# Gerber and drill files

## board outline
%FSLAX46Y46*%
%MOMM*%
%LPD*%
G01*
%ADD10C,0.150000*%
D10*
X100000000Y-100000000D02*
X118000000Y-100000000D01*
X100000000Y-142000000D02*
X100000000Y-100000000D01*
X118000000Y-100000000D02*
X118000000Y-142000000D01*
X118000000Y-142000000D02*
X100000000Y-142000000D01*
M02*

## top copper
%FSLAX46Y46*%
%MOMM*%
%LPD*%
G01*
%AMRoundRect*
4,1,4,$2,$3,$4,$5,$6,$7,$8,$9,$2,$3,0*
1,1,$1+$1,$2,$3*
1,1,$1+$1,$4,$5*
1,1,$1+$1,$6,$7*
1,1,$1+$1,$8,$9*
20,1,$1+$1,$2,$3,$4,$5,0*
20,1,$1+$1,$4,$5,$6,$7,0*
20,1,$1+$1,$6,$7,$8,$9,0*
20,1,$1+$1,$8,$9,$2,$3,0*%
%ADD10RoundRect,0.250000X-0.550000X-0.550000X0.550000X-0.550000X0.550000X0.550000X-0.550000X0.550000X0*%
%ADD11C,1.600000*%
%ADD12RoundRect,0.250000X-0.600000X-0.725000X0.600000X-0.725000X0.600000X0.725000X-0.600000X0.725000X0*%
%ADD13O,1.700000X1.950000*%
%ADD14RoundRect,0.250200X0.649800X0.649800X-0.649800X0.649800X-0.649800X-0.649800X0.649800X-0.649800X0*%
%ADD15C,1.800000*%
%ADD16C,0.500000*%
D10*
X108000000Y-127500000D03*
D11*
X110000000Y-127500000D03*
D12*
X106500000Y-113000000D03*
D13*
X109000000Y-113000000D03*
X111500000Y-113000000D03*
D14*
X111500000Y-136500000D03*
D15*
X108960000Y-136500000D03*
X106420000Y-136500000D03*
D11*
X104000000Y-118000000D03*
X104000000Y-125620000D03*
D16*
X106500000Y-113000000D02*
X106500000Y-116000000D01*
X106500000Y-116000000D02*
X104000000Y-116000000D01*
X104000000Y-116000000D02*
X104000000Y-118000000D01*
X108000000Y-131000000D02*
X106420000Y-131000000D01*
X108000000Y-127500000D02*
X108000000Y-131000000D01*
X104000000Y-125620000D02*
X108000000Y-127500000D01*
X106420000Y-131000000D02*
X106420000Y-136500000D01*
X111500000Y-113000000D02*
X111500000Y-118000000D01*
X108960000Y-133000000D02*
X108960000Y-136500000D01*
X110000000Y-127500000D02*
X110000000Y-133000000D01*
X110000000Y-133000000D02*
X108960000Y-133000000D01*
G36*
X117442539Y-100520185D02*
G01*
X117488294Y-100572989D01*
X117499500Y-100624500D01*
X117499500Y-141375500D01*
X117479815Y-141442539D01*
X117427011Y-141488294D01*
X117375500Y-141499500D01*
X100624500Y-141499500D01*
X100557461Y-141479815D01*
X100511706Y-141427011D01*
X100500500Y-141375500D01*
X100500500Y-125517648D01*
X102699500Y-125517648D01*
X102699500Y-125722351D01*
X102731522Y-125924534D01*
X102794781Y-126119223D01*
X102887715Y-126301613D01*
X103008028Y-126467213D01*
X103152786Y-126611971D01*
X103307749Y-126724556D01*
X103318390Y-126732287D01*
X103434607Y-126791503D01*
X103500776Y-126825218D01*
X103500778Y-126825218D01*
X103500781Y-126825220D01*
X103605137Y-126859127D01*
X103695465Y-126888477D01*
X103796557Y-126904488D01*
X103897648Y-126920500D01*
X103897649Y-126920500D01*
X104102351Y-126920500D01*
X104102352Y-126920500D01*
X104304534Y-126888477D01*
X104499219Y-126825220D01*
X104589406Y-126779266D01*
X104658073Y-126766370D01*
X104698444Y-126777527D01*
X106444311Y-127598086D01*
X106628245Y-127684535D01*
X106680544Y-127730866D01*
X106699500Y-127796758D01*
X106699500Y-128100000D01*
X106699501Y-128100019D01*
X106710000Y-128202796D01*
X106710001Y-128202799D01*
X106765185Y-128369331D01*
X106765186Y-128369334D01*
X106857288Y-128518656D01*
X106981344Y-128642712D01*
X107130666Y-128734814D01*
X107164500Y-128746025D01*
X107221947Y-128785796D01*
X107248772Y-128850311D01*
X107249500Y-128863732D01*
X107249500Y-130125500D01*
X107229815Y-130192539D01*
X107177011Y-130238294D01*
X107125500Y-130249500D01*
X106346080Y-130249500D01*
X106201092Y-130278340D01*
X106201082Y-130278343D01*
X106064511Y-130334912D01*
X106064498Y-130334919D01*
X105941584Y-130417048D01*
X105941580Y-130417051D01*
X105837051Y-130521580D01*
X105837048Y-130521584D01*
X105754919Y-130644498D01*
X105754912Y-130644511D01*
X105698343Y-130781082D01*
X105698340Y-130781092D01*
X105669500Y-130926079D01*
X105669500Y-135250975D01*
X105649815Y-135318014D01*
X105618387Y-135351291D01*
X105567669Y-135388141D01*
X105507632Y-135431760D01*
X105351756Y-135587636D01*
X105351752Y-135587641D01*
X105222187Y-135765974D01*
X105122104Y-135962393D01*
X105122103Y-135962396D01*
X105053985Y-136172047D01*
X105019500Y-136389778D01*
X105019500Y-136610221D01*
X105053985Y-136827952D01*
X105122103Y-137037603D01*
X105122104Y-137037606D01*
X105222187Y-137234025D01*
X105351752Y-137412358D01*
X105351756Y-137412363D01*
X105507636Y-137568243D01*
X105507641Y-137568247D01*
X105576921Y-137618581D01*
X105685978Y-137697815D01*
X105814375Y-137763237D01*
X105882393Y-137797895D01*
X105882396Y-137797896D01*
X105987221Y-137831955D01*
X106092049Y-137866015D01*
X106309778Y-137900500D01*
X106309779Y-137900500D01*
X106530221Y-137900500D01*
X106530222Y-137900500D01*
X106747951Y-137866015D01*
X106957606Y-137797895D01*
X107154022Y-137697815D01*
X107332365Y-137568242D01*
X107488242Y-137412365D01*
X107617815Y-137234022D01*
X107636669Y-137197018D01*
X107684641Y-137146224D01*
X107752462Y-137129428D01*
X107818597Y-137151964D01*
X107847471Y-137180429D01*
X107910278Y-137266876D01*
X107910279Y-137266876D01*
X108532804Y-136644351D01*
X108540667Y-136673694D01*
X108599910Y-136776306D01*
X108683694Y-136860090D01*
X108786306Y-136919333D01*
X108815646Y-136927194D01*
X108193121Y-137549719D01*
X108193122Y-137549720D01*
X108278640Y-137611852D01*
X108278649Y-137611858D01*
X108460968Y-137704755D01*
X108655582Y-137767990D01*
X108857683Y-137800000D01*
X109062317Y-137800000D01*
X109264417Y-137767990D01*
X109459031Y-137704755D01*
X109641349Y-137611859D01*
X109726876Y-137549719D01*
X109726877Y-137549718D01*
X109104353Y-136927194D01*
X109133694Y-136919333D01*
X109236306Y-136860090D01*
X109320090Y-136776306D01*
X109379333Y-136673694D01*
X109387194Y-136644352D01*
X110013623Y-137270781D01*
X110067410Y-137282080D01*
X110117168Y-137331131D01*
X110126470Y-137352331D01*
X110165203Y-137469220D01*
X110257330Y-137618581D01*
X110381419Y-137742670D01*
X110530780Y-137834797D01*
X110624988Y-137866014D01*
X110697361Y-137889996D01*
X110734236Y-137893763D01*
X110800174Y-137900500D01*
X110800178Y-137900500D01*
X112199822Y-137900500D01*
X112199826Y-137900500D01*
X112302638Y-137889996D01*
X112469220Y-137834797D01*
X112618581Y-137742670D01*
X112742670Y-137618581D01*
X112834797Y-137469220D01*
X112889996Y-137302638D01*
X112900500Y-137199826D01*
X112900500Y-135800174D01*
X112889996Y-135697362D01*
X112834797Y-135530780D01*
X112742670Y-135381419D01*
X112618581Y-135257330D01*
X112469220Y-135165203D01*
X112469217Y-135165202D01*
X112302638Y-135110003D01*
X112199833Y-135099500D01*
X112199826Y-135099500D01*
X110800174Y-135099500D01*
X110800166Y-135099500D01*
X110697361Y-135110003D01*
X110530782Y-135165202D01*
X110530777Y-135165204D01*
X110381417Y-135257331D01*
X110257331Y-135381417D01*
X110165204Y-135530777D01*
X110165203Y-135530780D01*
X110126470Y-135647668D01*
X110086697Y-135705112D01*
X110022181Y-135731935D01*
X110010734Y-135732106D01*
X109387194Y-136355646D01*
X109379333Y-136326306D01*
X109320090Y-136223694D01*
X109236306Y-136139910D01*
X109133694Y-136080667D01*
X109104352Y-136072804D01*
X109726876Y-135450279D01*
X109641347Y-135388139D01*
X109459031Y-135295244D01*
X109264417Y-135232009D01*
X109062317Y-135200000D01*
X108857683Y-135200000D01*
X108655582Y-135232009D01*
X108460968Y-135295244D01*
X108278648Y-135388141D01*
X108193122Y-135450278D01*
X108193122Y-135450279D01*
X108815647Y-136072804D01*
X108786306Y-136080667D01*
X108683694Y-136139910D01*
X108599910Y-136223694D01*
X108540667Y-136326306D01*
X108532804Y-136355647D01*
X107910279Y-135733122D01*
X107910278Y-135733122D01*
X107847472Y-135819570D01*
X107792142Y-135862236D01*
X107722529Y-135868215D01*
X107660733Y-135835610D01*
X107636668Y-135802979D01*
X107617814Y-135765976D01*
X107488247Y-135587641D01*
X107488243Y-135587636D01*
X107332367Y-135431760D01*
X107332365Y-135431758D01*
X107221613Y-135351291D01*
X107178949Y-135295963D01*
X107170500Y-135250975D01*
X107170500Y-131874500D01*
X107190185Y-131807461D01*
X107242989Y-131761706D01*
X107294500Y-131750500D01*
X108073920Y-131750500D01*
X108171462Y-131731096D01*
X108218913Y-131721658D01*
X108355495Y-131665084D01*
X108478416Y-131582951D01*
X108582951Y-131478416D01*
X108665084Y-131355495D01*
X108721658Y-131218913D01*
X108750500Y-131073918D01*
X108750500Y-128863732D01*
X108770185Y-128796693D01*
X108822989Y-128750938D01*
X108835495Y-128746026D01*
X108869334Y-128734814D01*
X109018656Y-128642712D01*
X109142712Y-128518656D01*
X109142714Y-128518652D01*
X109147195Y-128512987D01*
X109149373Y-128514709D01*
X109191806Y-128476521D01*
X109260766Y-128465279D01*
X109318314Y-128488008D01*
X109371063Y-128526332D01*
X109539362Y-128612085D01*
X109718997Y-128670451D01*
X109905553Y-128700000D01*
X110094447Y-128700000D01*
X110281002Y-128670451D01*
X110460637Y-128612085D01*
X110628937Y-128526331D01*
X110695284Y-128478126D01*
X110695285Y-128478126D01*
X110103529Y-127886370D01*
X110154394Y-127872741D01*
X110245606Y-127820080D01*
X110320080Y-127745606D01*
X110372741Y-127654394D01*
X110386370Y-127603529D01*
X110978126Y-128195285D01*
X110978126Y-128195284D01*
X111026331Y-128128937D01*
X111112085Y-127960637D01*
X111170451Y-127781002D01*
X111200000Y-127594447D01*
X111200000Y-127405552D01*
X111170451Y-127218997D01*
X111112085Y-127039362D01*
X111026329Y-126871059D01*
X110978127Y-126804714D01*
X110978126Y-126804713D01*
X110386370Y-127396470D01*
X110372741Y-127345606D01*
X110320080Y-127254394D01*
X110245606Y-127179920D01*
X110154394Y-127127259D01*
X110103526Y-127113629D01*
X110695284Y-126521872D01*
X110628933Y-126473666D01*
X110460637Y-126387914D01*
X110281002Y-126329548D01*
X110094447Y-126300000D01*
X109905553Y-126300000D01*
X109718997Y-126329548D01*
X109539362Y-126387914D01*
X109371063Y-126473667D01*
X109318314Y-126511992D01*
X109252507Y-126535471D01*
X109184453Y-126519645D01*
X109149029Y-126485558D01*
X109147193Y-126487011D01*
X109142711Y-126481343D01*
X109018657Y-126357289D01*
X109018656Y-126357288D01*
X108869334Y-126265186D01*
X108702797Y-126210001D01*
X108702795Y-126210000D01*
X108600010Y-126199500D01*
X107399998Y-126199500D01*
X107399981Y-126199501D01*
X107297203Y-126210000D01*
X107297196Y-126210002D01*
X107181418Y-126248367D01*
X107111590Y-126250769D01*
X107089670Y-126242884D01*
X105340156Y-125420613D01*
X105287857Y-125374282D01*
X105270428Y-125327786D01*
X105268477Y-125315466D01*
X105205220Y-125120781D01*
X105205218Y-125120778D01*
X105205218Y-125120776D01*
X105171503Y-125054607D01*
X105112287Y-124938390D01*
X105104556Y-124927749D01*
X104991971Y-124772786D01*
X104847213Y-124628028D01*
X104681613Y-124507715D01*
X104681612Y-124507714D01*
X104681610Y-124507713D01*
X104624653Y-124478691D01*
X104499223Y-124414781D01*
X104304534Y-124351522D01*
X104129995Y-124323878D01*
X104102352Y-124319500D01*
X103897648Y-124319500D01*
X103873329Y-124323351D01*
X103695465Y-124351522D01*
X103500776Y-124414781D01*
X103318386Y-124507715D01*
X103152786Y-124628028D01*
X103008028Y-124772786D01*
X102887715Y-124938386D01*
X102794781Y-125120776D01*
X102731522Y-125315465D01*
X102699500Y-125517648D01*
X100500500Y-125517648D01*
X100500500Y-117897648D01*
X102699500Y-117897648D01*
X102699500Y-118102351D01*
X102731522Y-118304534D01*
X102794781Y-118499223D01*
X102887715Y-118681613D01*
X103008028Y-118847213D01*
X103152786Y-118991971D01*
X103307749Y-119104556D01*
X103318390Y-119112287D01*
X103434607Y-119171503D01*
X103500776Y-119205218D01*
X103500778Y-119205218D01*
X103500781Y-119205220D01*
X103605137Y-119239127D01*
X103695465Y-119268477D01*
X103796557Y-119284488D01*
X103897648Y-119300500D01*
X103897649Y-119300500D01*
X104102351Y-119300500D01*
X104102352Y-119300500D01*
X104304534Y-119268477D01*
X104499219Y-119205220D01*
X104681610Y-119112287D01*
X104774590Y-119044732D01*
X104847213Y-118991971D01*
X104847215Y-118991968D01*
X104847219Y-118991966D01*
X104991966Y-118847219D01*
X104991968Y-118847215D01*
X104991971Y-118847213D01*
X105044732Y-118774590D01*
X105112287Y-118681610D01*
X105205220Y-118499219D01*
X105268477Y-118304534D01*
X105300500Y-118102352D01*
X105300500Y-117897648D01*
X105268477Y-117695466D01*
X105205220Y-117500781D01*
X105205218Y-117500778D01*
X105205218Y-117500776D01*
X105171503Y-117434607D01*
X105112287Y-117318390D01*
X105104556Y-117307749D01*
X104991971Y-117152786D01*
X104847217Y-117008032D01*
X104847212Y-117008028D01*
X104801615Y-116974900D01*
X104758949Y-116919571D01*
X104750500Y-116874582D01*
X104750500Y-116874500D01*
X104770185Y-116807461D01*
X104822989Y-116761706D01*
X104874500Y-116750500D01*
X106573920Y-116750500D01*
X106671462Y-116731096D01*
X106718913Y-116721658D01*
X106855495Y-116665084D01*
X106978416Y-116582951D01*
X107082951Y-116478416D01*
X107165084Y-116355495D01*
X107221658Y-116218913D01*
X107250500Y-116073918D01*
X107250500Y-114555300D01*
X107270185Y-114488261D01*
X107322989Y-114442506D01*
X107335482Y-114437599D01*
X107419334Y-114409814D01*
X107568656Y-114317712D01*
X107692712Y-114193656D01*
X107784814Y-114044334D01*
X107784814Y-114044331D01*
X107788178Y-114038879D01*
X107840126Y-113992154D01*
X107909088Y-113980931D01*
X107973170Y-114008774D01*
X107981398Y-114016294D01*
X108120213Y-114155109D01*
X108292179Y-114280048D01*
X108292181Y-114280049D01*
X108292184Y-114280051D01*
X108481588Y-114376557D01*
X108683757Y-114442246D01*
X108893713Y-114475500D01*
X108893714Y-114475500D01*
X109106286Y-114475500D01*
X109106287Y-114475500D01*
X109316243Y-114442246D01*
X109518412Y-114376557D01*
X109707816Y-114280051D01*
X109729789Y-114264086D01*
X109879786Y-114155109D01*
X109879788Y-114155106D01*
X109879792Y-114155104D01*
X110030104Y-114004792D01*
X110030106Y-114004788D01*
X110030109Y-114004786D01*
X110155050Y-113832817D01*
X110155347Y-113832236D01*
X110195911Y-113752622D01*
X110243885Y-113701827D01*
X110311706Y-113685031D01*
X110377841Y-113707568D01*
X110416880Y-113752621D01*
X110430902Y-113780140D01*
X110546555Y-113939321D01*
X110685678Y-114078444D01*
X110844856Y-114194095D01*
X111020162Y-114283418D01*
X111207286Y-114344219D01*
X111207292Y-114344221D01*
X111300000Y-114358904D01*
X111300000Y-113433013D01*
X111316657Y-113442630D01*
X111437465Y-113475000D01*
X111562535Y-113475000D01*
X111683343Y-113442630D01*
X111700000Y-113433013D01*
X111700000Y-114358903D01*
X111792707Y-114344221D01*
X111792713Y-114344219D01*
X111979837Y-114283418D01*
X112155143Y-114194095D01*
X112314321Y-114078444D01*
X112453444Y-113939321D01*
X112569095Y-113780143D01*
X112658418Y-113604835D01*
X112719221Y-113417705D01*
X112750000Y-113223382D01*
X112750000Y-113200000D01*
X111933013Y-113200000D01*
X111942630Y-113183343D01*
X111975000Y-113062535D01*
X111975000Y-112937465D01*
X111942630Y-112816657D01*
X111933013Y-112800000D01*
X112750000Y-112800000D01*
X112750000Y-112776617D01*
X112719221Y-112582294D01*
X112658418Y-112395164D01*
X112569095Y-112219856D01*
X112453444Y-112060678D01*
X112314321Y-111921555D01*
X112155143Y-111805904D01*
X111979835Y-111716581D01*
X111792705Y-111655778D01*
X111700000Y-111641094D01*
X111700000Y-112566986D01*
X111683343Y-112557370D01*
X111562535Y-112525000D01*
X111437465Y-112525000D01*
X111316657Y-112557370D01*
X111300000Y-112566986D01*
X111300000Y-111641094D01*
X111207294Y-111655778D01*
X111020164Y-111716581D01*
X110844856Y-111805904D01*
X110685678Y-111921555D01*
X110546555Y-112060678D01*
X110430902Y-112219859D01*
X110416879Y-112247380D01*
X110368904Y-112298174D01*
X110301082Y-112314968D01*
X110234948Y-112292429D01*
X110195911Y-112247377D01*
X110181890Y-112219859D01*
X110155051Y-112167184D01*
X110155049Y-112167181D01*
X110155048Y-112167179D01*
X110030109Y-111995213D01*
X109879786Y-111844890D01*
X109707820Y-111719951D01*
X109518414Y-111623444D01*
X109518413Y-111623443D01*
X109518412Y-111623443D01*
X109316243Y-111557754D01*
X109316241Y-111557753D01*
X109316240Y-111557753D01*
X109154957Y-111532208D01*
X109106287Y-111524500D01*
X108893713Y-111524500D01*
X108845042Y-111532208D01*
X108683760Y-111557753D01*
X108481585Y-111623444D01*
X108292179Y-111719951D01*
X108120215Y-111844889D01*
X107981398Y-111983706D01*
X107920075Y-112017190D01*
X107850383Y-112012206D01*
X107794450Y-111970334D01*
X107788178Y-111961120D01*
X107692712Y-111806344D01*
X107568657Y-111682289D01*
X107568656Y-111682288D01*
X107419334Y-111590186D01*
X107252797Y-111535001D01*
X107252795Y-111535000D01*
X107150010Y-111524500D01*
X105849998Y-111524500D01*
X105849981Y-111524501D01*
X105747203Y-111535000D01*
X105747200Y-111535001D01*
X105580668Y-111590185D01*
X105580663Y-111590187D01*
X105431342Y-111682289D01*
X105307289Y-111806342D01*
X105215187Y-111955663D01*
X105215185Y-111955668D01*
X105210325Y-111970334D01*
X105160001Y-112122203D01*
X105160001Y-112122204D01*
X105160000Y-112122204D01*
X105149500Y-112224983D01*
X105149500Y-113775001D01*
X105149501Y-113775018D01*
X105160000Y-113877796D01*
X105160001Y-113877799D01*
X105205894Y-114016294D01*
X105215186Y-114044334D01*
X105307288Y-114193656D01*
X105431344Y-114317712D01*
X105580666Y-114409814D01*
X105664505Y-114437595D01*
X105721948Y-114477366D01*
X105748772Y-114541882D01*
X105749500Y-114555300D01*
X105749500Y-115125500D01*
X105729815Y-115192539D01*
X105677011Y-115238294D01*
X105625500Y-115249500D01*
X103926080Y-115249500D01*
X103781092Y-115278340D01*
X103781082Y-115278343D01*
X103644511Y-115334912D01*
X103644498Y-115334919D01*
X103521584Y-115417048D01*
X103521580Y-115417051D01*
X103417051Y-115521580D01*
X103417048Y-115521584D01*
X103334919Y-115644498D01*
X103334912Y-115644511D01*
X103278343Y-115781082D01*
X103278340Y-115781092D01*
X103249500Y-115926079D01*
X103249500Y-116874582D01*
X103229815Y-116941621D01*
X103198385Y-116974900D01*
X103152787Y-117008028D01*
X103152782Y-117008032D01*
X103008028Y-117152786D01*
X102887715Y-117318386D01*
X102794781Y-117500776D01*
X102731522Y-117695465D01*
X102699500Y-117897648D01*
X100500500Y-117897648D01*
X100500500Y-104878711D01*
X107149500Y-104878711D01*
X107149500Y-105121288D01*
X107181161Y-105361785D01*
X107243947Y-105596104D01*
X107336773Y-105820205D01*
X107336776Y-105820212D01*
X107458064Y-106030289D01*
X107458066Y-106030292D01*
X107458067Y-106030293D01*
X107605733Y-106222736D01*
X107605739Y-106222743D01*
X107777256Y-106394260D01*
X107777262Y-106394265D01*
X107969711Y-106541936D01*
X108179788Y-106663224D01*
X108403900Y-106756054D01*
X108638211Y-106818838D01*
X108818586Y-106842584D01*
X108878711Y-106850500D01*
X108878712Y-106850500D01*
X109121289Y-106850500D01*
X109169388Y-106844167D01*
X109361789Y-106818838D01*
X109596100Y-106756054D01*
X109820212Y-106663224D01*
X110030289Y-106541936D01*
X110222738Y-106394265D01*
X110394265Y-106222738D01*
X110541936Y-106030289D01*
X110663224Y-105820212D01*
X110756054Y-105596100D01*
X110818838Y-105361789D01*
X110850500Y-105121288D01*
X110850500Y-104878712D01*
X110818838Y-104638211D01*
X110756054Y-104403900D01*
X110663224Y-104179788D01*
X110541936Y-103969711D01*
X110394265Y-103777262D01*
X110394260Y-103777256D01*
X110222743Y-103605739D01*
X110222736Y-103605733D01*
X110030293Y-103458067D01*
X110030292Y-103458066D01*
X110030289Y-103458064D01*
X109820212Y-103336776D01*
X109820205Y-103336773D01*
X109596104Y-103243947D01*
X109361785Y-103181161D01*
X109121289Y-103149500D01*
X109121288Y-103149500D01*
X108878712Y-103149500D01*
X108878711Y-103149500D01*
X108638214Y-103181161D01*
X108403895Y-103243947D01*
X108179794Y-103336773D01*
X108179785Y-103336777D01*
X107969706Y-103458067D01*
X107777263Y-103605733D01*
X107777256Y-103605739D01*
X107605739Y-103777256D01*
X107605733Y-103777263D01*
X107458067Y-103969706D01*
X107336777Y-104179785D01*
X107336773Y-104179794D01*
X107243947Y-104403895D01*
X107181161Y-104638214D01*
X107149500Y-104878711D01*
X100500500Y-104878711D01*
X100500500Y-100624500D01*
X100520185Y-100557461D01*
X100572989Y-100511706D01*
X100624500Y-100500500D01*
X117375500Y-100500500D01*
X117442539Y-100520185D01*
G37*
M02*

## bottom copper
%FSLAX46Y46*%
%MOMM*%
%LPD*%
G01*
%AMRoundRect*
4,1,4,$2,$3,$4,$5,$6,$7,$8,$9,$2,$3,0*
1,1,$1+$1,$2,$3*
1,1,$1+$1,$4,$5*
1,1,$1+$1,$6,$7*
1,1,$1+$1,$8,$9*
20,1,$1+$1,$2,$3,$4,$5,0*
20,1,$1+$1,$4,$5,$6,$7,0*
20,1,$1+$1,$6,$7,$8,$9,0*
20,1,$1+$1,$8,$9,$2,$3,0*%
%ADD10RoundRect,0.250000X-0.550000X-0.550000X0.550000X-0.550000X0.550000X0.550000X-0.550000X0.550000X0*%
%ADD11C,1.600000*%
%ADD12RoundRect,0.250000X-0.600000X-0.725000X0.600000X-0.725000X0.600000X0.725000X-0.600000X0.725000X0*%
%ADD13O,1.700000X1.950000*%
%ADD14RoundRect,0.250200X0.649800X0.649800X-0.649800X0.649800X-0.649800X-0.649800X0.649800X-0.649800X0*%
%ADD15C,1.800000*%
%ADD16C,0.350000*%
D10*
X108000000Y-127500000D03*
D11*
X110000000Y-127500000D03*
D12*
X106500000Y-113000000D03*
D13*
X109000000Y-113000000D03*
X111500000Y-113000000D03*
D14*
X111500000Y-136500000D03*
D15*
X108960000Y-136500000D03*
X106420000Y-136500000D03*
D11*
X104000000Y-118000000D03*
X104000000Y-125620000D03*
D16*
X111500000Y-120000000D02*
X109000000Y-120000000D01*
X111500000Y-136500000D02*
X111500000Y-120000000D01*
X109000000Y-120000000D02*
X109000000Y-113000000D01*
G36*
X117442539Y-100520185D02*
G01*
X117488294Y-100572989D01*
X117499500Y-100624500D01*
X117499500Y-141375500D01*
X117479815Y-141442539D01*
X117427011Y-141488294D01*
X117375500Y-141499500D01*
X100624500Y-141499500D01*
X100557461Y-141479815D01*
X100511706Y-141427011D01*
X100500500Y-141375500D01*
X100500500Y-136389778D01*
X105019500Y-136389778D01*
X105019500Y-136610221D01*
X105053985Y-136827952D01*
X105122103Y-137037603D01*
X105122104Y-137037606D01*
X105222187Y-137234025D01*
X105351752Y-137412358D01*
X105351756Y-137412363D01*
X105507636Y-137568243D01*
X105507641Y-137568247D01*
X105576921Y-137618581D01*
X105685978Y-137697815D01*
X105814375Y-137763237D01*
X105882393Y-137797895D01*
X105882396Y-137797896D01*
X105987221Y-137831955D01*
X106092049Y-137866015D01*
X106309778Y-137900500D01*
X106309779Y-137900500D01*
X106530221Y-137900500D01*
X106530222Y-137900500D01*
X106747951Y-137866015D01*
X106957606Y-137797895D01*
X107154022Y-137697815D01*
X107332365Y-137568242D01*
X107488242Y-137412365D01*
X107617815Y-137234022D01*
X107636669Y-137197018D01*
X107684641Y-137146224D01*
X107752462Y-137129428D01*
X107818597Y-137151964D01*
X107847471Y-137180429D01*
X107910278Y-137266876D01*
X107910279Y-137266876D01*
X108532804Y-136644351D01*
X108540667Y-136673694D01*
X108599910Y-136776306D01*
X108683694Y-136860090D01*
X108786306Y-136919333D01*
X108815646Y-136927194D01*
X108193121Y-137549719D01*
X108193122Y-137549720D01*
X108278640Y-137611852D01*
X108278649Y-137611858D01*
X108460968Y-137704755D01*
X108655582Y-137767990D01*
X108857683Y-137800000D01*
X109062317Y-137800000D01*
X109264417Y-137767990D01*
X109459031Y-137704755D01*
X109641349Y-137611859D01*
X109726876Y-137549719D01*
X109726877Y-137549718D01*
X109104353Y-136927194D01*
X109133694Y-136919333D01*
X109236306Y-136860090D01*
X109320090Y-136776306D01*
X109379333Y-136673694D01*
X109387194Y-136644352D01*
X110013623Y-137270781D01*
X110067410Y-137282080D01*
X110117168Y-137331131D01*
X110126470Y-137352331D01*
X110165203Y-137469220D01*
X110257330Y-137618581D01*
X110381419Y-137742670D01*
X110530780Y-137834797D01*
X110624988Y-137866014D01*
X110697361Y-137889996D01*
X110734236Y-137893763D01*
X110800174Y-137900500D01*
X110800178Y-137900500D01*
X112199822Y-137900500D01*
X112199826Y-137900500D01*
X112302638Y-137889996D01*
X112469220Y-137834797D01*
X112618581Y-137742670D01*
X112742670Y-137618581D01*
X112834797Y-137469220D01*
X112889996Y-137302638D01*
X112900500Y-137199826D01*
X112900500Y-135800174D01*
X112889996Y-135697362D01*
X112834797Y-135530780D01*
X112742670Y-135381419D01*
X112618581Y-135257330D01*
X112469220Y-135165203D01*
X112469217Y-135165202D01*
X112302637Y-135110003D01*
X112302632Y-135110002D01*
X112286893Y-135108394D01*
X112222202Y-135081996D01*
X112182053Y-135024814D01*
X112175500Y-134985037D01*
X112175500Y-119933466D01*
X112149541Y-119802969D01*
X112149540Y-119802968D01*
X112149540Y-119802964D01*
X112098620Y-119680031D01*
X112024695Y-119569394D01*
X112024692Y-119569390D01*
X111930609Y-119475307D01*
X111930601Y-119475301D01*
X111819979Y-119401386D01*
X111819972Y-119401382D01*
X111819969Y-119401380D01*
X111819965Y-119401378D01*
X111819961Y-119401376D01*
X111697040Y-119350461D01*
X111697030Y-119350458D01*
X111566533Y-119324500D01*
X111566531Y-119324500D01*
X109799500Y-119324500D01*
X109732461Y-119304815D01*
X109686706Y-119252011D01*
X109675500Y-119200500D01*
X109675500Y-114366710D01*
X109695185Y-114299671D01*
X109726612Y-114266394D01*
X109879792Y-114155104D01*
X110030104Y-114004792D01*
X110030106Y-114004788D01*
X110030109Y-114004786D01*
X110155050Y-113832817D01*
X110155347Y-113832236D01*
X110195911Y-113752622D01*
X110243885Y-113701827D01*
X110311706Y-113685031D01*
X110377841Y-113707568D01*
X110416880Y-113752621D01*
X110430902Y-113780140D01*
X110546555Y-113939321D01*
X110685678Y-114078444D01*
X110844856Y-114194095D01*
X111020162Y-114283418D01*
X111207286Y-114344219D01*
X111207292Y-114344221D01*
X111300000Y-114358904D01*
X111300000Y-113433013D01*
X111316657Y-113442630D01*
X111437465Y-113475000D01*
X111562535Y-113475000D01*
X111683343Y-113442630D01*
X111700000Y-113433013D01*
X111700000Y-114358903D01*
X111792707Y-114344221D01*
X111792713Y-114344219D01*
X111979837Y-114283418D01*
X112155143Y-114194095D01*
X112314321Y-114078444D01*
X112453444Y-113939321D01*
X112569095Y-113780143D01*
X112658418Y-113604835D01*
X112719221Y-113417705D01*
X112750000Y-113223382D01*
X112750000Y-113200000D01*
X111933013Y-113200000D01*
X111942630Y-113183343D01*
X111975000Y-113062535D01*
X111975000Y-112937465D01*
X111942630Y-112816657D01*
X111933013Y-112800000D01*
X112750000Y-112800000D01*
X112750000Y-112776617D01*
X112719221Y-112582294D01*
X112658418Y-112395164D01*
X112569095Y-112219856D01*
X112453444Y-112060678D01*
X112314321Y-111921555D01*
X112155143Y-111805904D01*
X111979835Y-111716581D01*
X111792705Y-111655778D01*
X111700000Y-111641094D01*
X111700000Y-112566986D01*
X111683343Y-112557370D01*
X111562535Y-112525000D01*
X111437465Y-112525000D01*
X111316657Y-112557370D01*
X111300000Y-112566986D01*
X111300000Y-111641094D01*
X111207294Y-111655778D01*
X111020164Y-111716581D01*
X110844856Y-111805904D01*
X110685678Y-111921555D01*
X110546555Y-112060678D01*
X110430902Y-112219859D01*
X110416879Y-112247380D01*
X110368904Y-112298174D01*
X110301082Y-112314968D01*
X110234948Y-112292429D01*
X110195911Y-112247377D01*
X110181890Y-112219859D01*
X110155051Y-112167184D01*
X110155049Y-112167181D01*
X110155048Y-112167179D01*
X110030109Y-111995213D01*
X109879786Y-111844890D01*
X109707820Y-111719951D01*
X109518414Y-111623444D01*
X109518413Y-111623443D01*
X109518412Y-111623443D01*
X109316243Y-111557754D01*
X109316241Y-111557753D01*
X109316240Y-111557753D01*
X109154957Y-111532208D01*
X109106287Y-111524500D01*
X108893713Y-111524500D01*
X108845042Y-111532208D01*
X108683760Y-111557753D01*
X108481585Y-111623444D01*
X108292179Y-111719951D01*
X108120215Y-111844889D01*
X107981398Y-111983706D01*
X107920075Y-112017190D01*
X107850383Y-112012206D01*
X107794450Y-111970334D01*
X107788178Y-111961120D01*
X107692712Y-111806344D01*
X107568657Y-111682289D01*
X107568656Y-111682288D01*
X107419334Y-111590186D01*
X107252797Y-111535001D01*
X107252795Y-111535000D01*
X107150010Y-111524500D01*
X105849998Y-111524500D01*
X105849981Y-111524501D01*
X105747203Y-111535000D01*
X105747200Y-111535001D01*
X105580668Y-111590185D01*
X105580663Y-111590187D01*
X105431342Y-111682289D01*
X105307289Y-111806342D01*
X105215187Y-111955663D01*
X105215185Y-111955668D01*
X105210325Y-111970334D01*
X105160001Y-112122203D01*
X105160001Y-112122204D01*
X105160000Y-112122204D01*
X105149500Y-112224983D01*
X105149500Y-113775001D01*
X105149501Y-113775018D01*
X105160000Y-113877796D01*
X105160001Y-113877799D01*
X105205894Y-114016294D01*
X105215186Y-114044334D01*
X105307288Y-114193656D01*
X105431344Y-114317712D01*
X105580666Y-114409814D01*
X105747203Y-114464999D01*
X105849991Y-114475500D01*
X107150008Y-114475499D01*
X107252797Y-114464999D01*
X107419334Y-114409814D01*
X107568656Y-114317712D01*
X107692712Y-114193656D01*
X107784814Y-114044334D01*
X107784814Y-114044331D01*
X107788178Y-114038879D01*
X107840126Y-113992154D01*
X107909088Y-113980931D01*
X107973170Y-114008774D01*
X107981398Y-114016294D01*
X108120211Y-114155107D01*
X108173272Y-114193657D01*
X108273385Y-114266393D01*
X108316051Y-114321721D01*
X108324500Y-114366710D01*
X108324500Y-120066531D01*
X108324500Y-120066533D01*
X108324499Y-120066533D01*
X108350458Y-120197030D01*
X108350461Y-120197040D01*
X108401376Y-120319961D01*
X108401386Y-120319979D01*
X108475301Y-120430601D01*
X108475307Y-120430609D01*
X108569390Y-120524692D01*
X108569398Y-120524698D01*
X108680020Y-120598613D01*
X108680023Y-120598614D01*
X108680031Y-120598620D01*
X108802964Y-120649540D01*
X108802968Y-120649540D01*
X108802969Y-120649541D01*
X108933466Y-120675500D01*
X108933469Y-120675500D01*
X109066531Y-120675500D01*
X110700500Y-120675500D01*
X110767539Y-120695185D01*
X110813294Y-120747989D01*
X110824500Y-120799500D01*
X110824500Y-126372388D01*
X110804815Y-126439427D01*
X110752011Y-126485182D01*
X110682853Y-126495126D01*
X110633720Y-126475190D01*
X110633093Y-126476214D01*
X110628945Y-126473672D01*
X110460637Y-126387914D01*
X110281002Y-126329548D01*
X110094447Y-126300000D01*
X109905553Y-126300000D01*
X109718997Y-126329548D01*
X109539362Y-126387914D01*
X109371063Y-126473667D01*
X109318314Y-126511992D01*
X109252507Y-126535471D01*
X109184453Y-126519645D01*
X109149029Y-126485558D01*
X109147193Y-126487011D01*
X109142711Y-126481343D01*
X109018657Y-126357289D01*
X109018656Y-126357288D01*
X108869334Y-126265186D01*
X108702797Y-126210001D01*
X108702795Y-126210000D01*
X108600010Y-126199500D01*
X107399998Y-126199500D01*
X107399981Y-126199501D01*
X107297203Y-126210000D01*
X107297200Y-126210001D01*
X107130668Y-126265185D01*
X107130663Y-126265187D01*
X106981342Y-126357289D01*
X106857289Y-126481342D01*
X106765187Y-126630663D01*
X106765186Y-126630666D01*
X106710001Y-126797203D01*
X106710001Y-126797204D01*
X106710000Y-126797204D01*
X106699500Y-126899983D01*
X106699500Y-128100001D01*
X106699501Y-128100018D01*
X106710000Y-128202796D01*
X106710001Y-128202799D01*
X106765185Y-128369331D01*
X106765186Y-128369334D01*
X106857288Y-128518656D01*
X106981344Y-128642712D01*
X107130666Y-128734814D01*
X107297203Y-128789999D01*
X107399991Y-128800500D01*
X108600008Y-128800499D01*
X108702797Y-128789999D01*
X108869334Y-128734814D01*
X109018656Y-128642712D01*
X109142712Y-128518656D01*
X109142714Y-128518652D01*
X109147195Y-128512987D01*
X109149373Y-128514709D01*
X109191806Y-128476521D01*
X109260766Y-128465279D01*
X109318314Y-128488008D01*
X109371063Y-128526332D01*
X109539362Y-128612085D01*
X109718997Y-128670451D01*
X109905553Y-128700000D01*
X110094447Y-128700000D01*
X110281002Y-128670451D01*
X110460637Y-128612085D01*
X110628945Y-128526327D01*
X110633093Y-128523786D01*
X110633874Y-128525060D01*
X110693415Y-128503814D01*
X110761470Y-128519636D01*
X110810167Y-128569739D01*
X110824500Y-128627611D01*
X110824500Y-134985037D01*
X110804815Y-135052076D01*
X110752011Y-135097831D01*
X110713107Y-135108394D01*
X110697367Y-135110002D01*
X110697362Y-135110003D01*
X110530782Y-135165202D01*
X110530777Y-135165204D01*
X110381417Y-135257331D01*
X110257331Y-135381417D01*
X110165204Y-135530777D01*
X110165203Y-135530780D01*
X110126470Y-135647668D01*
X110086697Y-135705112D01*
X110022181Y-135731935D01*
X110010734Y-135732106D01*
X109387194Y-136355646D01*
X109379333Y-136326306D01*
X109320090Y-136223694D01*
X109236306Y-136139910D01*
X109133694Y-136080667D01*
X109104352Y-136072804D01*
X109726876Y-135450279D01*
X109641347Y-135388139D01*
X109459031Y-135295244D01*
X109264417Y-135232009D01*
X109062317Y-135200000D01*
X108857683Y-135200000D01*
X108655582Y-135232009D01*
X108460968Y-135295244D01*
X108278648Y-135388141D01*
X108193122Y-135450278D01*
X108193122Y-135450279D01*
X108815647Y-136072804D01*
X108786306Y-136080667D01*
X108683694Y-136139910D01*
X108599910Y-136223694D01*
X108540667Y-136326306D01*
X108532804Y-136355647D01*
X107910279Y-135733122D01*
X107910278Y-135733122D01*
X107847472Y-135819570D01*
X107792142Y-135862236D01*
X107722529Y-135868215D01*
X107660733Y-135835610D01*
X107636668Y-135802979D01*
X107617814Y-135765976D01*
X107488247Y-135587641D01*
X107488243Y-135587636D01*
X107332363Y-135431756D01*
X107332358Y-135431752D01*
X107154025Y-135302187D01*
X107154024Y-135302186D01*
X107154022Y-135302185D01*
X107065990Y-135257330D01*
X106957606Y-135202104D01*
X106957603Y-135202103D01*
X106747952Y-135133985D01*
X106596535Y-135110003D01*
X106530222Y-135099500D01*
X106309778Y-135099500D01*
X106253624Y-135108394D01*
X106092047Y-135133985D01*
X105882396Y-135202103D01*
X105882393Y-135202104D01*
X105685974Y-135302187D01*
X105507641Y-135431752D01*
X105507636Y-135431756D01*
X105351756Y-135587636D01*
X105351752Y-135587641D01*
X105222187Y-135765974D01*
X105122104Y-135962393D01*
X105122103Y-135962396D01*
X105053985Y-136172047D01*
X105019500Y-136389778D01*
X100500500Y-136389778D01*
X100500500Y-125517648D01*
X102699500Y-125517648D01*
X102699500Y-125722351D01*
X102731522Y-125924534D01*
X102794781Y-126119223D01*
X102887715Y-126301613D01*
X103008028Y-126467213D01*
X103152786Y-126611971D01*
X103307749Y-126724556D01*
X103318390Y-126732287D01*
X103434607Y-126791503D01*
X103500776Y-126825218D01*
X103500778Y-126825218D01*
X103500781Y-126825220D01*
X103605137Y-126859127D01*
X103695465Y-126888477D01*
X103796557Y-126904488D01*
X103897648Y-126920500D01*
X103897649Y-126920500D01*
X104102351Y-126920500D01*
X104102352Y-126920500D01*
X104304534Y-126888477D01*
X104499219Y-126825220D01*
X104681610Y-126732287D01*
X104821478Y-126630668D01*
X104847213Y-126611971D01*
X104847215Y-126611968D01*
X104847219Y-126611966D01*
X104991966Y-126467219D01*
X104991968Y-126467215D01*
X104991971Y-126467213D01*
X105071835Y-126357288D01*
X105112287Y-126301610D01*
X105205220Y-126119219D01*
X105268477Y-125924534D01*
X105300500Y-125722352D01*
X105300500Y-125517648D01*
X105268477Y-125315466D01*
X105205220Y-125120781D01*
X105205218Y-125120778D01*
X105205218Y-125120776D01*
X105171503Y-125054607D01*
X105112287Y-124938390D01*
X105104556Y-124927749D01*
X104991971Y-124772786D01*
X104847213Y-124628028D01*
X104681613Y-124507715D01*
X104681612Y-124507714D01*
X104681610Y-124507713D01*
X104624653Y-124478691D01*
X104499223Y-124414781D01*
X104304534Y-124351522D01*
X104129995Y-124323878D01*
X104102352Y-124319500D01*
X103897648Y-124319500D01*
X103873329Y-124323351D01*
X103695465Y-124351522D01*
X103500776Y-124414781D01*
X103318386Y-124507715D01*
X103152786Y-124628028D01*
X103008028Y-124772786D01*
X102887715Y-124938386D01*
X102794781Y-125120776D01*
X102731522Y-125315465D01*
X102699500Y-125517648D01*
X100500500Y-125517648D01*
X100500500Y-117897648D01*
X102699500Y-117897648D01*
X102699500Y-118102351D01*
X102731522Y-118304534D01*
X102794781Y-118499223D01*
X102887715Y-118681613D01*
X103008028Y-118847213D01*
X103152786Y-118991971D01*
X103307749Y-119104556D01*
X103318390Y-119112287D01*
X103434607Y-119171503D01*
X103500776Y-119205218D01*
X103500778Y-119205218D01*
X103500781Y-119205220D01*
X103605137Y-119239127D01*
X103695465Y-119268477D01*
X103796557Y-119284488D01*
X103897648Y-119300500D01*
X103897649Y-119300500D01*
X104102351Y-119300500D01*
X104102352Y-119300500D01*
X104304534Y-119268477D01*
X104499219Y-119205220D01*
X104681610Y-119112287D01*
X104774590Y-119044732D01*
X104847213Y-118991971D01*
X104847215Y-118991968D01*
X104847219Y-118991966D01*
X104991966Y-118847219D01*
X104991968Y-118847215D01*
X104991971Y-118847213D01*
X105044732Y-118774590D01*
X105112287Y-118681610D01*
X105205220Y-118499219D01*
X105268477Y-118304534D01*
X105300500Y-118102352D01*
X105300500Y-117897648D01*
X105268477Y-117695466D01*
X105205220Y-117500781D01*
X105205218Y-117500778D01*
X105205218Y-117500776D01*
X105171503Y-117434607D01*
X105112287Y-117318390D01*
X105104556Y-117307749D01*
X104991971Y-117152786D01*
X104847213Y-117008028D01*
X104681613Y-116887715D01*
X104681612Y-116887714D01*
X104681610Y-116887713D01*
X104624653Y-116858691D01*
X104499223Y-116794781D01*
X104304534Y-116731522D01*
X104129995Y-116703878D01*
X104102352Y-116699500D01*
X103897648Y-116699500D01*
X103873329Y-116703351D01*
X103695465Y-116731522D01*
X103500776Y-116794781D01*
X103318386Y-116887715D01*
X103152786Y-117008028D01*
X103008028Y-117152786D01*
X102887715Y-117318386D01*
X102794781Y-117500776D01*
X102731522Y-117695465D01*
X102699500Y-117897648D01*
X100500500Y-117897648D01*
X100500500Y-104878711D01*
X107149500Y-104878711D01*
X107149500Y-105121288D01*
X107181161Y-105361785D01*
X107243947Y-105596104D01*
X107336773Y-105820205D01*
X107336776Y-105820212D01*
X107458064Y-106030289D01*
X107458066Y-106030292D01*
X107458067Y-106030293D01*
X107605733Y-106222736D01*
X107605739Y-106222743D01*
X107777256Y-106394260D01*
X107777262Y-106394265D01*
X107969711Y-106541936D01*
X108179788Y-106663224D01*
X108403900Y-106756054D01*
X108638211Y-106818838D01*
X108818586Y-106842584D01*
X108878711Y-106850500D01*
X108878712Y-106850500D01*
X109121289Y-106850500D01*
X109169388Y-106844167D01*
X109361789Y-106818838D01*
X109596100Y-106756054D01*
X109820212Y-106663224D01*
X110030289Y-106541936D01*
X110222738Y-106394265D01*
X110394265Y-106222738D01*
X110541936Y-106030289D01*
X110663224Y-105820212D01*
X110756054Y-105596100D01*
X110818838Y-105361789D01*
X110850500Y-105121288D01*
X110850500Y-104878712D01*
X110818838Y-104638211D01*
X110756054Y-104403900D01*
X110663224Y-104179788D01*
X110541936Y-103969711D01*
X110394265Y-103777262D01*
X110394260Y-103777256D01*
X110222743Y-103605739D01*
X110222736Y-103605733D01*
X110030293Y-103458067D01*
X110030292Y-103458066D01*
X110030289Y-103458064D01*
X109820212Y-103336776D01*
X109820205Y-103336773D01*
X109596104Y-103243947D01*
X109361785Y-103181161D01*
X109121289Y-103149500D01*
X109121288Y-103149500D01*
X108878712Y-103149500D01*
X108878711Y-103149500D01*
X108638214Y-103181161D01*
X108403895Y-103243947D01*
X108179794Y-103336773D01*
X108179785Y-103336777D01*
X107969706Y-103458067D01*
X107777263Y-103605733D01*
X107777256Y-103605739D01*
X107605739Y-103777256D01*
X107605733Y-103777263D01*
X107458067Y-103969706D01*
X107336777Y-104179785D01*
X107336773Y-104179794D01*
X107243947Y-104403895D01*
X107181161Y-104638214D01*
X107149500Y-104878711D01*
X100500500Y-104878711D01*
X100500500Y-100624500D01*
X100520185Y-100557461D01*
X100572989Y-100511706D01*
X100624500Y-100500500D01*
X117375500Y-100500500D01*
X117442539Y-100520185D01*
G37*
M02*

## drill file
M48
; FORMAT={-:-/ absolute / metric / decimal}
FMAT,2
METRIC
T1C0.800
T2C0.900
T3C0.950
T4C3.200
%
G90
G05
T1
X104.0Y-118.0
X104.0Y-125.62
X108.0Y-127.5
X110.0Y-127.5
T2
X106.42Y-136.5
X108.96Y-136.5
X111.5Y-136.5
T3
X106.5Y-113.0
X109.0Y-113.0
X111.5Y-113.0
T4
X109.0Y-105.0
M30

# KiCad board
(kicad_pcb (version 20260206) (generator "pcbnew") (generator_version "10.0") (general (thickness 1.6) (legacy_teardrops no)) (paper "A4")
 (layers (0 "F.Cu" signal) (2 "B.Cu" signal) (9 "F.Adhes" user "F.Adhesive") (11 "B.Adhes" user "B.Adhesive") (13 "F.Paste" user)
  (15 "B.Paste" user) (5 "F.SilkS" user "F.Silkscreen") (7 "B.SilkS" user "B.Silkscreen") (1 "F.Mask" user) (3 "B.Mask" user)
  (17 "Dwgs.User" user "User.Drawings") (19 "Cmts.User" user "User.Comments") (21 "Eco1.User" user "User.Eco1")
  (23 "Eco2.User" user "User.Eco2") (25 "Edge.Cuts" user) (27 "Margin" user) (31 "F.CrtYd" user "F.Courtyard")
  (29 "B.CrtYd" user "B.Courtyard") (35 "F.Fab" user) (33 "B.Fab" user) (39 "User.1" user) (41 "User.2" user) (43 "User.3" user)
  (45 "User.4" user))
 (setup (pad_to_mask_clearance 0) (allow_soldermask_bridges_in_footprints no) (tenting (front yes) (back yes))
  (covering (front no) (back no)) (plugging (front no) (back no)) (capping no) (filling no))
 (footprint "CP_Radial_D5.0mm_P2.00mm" (layer "F.Cu") (at 108 127.5)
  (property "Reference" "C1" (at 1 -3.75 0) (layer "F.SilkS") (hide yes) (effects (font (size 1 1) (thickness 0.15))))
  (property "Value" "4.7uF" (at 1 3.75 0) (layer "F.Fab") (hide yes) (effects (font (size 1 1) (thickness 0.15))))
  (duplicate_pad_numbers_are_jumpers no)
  (pad "1" thru_hole roundrect (at 0 0) (size 1.6 1.6) (drill 0.8) (layers "*.Cu" "*.Mask") (remove_unused_layers no)
   (roundrect_rratio 0.15625) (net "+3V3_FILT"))
  (pad "2" thru_hole circle (at 2 0) (size 1.6 1.6) (drill 0.8) (layers "*.Cu" "*.Mask") (remove_unused_layers no) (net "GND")))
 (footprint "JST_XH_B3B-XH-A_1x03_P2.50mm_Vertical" (layer "F.Cu") (at 106.5 113)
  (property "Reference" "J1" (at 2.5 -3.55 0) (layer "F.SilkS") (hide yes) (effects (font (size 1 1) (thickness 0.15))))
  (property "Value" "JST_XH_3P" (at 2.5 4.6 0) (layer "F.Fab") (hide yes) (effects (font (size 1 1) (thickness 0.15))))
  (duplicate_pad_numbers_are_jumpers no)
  (pad "1" thru_hole roundrect (at 0 0) (size 1.7 1.95) (drill 0.95) (layers "*.Cu" "*.Mask") (remove_unused_layers no)
   (roundrect_rratio 0.147059) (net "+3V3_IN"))
  (pad "2" thru_hole oval (at 2.5 0) (size 1.7 1.95) (drill 0.95) (layers "*.Cu" "*.Mask") (remove_unused_layers no) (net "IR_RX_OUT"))
  (pad "3" thru_hole oval (at 5 0) (size 1.7 1.95) (drill 0.95) (layers "*.Cu" "*.Mask") (remove_unused_layers no) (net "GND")))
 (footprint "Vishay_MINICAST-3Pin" (layer "F.Cu") (at 111.5 136.5 180)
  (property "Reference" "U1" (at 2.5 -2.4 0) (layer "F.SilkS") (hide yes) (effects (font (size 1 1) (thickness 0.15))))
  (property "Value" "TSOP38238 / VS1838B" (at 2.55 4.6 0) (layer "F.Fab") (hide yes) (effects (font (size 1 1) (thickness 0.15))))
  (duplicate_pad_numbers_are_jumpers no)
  (pad "1" thru_hole roundrect (at 0 0 180) (size 1.8 1.8) (drill 0.9) (layers "*.Cu" "*.Mask") (remove_unused_layers no)
   (roundrect_rratio 0.139) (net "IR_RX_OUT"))
  (pad "2" thru_hole circle (at 2.54 0 180) (size 1.8 1.8) (drill 0.9) (layers "*.Cu" "*.Mask") (remove_unused_layers no) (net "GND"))
  (pad "3" thru_hole circle (at 5.08 0 180) (size 1.8 1.8) (drill 0.9) (layers "*.Cu" "*.Mask") (remove_unused_layers no) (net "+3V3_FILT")))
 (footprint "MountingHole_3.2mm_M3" (layer "F.Cu") (at 109 105)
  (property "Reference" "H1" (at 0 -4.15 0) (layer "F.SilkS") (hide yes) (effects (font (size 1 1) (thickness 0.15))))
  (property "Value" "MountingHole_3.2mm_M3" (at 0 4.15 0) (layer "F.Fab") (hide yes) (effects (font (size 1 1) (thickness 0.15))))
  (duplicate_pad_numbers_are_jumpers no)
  (pad "" np_thru_hole circle (at 0 0) (size 3.2 3.2) (drill 3.2) (layers "*.Cu" "*.Mask")))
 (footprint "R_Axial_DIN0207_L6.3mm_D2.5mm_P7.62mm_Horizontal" (layer "F.Cu") (at 104 118 -90)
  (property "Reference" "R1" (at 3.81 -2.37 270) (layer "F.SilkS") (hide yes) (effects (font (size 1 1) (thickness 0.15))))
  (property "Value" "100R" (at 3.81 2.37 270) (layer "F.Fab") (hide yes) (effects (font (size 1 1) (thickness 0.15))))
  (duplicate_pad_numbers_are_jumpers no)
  (pad "1" thru_hole circle (at 0 0 270) (size 1.6 1.6) (drill 0.8) (layers "*.Cu" "*.Mask") (remove_unused_layers no) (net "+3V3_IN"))
  (pad "2" thru_hole circle (at 7.62 0 270) (size 1.6 1.6) (drill 0.8) (layers "*.Cu" "*.Mask") (remove_unused_layers no) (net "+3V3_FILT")))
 (gr_line (start 100 100) (end 118 100) (stroke (width 0.15) (type default)) (layer "Edge.Cuts"))
 (gr_line (start 100 142) (end 100 100) (stroke (width 0.15) (type default)) (layer "Edge.Cuts"))
 (gr_line (start 118 100) (end 118 142) (stroke (width 0.15) (type default)) (layer "Edge.Cuts"))
 (gr_line (start 118 142) (end 100 142) (stroke (width 0.15) (type default)) (layer "Edge.Cuts"))
 (segment (start 106.5 113) (end 106.5 116) (width 0.5) (layer "F.Cu") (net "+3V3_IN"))
 (segment (start 106.5 116) (end 104 116) (width 0.5) (layer "F.Cu") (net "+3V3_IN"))
 (segment (start 104 116) (end 104 118) (width 0.5) (layer "F.Cu") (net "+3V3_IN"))
 (segment (start 108 131) (end 106.42 131) (width 0.5) (layer "F.Cu") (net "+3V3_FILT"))
 (segment (start 108 127.5) (end 108 131) (width 0.5) (layer "F.Cu") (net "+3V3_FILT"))
 (segment (start 104 125.62) (end 108 127.5) (width 0.5) (layer "F.Cu") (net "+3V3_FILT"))
 (segment (start 106.42 131) (end 106.42 136.5) (width 0.5) (layer "F.Cu") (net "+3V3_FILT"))
 (segment (start 111.5 120) (end 109 120) (width 0.35) (layer "B.Cu") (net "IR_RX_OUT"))
 (segment (start 111.5 136.5) (end 111.5 120) (width 0.35) (layer "B.Cu") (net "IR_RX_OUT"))
 (segment (start 109 120) (end 109 113) (width 0.35) (layer "B.Cu") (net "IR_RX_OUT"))
 (segment (start 111.5 113) (end 111.5 118) (width 0.5) (layer "F.Cu") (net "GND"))
 (segment (start 108.96 133) (end 108.96 136.5) (width 0.5) (layer "F.Cu") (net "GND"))
 (segment (start 110 127.5) (end 110 133) (width 0.5) (layer "F.Cu") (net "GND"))
 (segment (start 110 133) (end 108.96 133) (width 0.5) (layer "F.Cu") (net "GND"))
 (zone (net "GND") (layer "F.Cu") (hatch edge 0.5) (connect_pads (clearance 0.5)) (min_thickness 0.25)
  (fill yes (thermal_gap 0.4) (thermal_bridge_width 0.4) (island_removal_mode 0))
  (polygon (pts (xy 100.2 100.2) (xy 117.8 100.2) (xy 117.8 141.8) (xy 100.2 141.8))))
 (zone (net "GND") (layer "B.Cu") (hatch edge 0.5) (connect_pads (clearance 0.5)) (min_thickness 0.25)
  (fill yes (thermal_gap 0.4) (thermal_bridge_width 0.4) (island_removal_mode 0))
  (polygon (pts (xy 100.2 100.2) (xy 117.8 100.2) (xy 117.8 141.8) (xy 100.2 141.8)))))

